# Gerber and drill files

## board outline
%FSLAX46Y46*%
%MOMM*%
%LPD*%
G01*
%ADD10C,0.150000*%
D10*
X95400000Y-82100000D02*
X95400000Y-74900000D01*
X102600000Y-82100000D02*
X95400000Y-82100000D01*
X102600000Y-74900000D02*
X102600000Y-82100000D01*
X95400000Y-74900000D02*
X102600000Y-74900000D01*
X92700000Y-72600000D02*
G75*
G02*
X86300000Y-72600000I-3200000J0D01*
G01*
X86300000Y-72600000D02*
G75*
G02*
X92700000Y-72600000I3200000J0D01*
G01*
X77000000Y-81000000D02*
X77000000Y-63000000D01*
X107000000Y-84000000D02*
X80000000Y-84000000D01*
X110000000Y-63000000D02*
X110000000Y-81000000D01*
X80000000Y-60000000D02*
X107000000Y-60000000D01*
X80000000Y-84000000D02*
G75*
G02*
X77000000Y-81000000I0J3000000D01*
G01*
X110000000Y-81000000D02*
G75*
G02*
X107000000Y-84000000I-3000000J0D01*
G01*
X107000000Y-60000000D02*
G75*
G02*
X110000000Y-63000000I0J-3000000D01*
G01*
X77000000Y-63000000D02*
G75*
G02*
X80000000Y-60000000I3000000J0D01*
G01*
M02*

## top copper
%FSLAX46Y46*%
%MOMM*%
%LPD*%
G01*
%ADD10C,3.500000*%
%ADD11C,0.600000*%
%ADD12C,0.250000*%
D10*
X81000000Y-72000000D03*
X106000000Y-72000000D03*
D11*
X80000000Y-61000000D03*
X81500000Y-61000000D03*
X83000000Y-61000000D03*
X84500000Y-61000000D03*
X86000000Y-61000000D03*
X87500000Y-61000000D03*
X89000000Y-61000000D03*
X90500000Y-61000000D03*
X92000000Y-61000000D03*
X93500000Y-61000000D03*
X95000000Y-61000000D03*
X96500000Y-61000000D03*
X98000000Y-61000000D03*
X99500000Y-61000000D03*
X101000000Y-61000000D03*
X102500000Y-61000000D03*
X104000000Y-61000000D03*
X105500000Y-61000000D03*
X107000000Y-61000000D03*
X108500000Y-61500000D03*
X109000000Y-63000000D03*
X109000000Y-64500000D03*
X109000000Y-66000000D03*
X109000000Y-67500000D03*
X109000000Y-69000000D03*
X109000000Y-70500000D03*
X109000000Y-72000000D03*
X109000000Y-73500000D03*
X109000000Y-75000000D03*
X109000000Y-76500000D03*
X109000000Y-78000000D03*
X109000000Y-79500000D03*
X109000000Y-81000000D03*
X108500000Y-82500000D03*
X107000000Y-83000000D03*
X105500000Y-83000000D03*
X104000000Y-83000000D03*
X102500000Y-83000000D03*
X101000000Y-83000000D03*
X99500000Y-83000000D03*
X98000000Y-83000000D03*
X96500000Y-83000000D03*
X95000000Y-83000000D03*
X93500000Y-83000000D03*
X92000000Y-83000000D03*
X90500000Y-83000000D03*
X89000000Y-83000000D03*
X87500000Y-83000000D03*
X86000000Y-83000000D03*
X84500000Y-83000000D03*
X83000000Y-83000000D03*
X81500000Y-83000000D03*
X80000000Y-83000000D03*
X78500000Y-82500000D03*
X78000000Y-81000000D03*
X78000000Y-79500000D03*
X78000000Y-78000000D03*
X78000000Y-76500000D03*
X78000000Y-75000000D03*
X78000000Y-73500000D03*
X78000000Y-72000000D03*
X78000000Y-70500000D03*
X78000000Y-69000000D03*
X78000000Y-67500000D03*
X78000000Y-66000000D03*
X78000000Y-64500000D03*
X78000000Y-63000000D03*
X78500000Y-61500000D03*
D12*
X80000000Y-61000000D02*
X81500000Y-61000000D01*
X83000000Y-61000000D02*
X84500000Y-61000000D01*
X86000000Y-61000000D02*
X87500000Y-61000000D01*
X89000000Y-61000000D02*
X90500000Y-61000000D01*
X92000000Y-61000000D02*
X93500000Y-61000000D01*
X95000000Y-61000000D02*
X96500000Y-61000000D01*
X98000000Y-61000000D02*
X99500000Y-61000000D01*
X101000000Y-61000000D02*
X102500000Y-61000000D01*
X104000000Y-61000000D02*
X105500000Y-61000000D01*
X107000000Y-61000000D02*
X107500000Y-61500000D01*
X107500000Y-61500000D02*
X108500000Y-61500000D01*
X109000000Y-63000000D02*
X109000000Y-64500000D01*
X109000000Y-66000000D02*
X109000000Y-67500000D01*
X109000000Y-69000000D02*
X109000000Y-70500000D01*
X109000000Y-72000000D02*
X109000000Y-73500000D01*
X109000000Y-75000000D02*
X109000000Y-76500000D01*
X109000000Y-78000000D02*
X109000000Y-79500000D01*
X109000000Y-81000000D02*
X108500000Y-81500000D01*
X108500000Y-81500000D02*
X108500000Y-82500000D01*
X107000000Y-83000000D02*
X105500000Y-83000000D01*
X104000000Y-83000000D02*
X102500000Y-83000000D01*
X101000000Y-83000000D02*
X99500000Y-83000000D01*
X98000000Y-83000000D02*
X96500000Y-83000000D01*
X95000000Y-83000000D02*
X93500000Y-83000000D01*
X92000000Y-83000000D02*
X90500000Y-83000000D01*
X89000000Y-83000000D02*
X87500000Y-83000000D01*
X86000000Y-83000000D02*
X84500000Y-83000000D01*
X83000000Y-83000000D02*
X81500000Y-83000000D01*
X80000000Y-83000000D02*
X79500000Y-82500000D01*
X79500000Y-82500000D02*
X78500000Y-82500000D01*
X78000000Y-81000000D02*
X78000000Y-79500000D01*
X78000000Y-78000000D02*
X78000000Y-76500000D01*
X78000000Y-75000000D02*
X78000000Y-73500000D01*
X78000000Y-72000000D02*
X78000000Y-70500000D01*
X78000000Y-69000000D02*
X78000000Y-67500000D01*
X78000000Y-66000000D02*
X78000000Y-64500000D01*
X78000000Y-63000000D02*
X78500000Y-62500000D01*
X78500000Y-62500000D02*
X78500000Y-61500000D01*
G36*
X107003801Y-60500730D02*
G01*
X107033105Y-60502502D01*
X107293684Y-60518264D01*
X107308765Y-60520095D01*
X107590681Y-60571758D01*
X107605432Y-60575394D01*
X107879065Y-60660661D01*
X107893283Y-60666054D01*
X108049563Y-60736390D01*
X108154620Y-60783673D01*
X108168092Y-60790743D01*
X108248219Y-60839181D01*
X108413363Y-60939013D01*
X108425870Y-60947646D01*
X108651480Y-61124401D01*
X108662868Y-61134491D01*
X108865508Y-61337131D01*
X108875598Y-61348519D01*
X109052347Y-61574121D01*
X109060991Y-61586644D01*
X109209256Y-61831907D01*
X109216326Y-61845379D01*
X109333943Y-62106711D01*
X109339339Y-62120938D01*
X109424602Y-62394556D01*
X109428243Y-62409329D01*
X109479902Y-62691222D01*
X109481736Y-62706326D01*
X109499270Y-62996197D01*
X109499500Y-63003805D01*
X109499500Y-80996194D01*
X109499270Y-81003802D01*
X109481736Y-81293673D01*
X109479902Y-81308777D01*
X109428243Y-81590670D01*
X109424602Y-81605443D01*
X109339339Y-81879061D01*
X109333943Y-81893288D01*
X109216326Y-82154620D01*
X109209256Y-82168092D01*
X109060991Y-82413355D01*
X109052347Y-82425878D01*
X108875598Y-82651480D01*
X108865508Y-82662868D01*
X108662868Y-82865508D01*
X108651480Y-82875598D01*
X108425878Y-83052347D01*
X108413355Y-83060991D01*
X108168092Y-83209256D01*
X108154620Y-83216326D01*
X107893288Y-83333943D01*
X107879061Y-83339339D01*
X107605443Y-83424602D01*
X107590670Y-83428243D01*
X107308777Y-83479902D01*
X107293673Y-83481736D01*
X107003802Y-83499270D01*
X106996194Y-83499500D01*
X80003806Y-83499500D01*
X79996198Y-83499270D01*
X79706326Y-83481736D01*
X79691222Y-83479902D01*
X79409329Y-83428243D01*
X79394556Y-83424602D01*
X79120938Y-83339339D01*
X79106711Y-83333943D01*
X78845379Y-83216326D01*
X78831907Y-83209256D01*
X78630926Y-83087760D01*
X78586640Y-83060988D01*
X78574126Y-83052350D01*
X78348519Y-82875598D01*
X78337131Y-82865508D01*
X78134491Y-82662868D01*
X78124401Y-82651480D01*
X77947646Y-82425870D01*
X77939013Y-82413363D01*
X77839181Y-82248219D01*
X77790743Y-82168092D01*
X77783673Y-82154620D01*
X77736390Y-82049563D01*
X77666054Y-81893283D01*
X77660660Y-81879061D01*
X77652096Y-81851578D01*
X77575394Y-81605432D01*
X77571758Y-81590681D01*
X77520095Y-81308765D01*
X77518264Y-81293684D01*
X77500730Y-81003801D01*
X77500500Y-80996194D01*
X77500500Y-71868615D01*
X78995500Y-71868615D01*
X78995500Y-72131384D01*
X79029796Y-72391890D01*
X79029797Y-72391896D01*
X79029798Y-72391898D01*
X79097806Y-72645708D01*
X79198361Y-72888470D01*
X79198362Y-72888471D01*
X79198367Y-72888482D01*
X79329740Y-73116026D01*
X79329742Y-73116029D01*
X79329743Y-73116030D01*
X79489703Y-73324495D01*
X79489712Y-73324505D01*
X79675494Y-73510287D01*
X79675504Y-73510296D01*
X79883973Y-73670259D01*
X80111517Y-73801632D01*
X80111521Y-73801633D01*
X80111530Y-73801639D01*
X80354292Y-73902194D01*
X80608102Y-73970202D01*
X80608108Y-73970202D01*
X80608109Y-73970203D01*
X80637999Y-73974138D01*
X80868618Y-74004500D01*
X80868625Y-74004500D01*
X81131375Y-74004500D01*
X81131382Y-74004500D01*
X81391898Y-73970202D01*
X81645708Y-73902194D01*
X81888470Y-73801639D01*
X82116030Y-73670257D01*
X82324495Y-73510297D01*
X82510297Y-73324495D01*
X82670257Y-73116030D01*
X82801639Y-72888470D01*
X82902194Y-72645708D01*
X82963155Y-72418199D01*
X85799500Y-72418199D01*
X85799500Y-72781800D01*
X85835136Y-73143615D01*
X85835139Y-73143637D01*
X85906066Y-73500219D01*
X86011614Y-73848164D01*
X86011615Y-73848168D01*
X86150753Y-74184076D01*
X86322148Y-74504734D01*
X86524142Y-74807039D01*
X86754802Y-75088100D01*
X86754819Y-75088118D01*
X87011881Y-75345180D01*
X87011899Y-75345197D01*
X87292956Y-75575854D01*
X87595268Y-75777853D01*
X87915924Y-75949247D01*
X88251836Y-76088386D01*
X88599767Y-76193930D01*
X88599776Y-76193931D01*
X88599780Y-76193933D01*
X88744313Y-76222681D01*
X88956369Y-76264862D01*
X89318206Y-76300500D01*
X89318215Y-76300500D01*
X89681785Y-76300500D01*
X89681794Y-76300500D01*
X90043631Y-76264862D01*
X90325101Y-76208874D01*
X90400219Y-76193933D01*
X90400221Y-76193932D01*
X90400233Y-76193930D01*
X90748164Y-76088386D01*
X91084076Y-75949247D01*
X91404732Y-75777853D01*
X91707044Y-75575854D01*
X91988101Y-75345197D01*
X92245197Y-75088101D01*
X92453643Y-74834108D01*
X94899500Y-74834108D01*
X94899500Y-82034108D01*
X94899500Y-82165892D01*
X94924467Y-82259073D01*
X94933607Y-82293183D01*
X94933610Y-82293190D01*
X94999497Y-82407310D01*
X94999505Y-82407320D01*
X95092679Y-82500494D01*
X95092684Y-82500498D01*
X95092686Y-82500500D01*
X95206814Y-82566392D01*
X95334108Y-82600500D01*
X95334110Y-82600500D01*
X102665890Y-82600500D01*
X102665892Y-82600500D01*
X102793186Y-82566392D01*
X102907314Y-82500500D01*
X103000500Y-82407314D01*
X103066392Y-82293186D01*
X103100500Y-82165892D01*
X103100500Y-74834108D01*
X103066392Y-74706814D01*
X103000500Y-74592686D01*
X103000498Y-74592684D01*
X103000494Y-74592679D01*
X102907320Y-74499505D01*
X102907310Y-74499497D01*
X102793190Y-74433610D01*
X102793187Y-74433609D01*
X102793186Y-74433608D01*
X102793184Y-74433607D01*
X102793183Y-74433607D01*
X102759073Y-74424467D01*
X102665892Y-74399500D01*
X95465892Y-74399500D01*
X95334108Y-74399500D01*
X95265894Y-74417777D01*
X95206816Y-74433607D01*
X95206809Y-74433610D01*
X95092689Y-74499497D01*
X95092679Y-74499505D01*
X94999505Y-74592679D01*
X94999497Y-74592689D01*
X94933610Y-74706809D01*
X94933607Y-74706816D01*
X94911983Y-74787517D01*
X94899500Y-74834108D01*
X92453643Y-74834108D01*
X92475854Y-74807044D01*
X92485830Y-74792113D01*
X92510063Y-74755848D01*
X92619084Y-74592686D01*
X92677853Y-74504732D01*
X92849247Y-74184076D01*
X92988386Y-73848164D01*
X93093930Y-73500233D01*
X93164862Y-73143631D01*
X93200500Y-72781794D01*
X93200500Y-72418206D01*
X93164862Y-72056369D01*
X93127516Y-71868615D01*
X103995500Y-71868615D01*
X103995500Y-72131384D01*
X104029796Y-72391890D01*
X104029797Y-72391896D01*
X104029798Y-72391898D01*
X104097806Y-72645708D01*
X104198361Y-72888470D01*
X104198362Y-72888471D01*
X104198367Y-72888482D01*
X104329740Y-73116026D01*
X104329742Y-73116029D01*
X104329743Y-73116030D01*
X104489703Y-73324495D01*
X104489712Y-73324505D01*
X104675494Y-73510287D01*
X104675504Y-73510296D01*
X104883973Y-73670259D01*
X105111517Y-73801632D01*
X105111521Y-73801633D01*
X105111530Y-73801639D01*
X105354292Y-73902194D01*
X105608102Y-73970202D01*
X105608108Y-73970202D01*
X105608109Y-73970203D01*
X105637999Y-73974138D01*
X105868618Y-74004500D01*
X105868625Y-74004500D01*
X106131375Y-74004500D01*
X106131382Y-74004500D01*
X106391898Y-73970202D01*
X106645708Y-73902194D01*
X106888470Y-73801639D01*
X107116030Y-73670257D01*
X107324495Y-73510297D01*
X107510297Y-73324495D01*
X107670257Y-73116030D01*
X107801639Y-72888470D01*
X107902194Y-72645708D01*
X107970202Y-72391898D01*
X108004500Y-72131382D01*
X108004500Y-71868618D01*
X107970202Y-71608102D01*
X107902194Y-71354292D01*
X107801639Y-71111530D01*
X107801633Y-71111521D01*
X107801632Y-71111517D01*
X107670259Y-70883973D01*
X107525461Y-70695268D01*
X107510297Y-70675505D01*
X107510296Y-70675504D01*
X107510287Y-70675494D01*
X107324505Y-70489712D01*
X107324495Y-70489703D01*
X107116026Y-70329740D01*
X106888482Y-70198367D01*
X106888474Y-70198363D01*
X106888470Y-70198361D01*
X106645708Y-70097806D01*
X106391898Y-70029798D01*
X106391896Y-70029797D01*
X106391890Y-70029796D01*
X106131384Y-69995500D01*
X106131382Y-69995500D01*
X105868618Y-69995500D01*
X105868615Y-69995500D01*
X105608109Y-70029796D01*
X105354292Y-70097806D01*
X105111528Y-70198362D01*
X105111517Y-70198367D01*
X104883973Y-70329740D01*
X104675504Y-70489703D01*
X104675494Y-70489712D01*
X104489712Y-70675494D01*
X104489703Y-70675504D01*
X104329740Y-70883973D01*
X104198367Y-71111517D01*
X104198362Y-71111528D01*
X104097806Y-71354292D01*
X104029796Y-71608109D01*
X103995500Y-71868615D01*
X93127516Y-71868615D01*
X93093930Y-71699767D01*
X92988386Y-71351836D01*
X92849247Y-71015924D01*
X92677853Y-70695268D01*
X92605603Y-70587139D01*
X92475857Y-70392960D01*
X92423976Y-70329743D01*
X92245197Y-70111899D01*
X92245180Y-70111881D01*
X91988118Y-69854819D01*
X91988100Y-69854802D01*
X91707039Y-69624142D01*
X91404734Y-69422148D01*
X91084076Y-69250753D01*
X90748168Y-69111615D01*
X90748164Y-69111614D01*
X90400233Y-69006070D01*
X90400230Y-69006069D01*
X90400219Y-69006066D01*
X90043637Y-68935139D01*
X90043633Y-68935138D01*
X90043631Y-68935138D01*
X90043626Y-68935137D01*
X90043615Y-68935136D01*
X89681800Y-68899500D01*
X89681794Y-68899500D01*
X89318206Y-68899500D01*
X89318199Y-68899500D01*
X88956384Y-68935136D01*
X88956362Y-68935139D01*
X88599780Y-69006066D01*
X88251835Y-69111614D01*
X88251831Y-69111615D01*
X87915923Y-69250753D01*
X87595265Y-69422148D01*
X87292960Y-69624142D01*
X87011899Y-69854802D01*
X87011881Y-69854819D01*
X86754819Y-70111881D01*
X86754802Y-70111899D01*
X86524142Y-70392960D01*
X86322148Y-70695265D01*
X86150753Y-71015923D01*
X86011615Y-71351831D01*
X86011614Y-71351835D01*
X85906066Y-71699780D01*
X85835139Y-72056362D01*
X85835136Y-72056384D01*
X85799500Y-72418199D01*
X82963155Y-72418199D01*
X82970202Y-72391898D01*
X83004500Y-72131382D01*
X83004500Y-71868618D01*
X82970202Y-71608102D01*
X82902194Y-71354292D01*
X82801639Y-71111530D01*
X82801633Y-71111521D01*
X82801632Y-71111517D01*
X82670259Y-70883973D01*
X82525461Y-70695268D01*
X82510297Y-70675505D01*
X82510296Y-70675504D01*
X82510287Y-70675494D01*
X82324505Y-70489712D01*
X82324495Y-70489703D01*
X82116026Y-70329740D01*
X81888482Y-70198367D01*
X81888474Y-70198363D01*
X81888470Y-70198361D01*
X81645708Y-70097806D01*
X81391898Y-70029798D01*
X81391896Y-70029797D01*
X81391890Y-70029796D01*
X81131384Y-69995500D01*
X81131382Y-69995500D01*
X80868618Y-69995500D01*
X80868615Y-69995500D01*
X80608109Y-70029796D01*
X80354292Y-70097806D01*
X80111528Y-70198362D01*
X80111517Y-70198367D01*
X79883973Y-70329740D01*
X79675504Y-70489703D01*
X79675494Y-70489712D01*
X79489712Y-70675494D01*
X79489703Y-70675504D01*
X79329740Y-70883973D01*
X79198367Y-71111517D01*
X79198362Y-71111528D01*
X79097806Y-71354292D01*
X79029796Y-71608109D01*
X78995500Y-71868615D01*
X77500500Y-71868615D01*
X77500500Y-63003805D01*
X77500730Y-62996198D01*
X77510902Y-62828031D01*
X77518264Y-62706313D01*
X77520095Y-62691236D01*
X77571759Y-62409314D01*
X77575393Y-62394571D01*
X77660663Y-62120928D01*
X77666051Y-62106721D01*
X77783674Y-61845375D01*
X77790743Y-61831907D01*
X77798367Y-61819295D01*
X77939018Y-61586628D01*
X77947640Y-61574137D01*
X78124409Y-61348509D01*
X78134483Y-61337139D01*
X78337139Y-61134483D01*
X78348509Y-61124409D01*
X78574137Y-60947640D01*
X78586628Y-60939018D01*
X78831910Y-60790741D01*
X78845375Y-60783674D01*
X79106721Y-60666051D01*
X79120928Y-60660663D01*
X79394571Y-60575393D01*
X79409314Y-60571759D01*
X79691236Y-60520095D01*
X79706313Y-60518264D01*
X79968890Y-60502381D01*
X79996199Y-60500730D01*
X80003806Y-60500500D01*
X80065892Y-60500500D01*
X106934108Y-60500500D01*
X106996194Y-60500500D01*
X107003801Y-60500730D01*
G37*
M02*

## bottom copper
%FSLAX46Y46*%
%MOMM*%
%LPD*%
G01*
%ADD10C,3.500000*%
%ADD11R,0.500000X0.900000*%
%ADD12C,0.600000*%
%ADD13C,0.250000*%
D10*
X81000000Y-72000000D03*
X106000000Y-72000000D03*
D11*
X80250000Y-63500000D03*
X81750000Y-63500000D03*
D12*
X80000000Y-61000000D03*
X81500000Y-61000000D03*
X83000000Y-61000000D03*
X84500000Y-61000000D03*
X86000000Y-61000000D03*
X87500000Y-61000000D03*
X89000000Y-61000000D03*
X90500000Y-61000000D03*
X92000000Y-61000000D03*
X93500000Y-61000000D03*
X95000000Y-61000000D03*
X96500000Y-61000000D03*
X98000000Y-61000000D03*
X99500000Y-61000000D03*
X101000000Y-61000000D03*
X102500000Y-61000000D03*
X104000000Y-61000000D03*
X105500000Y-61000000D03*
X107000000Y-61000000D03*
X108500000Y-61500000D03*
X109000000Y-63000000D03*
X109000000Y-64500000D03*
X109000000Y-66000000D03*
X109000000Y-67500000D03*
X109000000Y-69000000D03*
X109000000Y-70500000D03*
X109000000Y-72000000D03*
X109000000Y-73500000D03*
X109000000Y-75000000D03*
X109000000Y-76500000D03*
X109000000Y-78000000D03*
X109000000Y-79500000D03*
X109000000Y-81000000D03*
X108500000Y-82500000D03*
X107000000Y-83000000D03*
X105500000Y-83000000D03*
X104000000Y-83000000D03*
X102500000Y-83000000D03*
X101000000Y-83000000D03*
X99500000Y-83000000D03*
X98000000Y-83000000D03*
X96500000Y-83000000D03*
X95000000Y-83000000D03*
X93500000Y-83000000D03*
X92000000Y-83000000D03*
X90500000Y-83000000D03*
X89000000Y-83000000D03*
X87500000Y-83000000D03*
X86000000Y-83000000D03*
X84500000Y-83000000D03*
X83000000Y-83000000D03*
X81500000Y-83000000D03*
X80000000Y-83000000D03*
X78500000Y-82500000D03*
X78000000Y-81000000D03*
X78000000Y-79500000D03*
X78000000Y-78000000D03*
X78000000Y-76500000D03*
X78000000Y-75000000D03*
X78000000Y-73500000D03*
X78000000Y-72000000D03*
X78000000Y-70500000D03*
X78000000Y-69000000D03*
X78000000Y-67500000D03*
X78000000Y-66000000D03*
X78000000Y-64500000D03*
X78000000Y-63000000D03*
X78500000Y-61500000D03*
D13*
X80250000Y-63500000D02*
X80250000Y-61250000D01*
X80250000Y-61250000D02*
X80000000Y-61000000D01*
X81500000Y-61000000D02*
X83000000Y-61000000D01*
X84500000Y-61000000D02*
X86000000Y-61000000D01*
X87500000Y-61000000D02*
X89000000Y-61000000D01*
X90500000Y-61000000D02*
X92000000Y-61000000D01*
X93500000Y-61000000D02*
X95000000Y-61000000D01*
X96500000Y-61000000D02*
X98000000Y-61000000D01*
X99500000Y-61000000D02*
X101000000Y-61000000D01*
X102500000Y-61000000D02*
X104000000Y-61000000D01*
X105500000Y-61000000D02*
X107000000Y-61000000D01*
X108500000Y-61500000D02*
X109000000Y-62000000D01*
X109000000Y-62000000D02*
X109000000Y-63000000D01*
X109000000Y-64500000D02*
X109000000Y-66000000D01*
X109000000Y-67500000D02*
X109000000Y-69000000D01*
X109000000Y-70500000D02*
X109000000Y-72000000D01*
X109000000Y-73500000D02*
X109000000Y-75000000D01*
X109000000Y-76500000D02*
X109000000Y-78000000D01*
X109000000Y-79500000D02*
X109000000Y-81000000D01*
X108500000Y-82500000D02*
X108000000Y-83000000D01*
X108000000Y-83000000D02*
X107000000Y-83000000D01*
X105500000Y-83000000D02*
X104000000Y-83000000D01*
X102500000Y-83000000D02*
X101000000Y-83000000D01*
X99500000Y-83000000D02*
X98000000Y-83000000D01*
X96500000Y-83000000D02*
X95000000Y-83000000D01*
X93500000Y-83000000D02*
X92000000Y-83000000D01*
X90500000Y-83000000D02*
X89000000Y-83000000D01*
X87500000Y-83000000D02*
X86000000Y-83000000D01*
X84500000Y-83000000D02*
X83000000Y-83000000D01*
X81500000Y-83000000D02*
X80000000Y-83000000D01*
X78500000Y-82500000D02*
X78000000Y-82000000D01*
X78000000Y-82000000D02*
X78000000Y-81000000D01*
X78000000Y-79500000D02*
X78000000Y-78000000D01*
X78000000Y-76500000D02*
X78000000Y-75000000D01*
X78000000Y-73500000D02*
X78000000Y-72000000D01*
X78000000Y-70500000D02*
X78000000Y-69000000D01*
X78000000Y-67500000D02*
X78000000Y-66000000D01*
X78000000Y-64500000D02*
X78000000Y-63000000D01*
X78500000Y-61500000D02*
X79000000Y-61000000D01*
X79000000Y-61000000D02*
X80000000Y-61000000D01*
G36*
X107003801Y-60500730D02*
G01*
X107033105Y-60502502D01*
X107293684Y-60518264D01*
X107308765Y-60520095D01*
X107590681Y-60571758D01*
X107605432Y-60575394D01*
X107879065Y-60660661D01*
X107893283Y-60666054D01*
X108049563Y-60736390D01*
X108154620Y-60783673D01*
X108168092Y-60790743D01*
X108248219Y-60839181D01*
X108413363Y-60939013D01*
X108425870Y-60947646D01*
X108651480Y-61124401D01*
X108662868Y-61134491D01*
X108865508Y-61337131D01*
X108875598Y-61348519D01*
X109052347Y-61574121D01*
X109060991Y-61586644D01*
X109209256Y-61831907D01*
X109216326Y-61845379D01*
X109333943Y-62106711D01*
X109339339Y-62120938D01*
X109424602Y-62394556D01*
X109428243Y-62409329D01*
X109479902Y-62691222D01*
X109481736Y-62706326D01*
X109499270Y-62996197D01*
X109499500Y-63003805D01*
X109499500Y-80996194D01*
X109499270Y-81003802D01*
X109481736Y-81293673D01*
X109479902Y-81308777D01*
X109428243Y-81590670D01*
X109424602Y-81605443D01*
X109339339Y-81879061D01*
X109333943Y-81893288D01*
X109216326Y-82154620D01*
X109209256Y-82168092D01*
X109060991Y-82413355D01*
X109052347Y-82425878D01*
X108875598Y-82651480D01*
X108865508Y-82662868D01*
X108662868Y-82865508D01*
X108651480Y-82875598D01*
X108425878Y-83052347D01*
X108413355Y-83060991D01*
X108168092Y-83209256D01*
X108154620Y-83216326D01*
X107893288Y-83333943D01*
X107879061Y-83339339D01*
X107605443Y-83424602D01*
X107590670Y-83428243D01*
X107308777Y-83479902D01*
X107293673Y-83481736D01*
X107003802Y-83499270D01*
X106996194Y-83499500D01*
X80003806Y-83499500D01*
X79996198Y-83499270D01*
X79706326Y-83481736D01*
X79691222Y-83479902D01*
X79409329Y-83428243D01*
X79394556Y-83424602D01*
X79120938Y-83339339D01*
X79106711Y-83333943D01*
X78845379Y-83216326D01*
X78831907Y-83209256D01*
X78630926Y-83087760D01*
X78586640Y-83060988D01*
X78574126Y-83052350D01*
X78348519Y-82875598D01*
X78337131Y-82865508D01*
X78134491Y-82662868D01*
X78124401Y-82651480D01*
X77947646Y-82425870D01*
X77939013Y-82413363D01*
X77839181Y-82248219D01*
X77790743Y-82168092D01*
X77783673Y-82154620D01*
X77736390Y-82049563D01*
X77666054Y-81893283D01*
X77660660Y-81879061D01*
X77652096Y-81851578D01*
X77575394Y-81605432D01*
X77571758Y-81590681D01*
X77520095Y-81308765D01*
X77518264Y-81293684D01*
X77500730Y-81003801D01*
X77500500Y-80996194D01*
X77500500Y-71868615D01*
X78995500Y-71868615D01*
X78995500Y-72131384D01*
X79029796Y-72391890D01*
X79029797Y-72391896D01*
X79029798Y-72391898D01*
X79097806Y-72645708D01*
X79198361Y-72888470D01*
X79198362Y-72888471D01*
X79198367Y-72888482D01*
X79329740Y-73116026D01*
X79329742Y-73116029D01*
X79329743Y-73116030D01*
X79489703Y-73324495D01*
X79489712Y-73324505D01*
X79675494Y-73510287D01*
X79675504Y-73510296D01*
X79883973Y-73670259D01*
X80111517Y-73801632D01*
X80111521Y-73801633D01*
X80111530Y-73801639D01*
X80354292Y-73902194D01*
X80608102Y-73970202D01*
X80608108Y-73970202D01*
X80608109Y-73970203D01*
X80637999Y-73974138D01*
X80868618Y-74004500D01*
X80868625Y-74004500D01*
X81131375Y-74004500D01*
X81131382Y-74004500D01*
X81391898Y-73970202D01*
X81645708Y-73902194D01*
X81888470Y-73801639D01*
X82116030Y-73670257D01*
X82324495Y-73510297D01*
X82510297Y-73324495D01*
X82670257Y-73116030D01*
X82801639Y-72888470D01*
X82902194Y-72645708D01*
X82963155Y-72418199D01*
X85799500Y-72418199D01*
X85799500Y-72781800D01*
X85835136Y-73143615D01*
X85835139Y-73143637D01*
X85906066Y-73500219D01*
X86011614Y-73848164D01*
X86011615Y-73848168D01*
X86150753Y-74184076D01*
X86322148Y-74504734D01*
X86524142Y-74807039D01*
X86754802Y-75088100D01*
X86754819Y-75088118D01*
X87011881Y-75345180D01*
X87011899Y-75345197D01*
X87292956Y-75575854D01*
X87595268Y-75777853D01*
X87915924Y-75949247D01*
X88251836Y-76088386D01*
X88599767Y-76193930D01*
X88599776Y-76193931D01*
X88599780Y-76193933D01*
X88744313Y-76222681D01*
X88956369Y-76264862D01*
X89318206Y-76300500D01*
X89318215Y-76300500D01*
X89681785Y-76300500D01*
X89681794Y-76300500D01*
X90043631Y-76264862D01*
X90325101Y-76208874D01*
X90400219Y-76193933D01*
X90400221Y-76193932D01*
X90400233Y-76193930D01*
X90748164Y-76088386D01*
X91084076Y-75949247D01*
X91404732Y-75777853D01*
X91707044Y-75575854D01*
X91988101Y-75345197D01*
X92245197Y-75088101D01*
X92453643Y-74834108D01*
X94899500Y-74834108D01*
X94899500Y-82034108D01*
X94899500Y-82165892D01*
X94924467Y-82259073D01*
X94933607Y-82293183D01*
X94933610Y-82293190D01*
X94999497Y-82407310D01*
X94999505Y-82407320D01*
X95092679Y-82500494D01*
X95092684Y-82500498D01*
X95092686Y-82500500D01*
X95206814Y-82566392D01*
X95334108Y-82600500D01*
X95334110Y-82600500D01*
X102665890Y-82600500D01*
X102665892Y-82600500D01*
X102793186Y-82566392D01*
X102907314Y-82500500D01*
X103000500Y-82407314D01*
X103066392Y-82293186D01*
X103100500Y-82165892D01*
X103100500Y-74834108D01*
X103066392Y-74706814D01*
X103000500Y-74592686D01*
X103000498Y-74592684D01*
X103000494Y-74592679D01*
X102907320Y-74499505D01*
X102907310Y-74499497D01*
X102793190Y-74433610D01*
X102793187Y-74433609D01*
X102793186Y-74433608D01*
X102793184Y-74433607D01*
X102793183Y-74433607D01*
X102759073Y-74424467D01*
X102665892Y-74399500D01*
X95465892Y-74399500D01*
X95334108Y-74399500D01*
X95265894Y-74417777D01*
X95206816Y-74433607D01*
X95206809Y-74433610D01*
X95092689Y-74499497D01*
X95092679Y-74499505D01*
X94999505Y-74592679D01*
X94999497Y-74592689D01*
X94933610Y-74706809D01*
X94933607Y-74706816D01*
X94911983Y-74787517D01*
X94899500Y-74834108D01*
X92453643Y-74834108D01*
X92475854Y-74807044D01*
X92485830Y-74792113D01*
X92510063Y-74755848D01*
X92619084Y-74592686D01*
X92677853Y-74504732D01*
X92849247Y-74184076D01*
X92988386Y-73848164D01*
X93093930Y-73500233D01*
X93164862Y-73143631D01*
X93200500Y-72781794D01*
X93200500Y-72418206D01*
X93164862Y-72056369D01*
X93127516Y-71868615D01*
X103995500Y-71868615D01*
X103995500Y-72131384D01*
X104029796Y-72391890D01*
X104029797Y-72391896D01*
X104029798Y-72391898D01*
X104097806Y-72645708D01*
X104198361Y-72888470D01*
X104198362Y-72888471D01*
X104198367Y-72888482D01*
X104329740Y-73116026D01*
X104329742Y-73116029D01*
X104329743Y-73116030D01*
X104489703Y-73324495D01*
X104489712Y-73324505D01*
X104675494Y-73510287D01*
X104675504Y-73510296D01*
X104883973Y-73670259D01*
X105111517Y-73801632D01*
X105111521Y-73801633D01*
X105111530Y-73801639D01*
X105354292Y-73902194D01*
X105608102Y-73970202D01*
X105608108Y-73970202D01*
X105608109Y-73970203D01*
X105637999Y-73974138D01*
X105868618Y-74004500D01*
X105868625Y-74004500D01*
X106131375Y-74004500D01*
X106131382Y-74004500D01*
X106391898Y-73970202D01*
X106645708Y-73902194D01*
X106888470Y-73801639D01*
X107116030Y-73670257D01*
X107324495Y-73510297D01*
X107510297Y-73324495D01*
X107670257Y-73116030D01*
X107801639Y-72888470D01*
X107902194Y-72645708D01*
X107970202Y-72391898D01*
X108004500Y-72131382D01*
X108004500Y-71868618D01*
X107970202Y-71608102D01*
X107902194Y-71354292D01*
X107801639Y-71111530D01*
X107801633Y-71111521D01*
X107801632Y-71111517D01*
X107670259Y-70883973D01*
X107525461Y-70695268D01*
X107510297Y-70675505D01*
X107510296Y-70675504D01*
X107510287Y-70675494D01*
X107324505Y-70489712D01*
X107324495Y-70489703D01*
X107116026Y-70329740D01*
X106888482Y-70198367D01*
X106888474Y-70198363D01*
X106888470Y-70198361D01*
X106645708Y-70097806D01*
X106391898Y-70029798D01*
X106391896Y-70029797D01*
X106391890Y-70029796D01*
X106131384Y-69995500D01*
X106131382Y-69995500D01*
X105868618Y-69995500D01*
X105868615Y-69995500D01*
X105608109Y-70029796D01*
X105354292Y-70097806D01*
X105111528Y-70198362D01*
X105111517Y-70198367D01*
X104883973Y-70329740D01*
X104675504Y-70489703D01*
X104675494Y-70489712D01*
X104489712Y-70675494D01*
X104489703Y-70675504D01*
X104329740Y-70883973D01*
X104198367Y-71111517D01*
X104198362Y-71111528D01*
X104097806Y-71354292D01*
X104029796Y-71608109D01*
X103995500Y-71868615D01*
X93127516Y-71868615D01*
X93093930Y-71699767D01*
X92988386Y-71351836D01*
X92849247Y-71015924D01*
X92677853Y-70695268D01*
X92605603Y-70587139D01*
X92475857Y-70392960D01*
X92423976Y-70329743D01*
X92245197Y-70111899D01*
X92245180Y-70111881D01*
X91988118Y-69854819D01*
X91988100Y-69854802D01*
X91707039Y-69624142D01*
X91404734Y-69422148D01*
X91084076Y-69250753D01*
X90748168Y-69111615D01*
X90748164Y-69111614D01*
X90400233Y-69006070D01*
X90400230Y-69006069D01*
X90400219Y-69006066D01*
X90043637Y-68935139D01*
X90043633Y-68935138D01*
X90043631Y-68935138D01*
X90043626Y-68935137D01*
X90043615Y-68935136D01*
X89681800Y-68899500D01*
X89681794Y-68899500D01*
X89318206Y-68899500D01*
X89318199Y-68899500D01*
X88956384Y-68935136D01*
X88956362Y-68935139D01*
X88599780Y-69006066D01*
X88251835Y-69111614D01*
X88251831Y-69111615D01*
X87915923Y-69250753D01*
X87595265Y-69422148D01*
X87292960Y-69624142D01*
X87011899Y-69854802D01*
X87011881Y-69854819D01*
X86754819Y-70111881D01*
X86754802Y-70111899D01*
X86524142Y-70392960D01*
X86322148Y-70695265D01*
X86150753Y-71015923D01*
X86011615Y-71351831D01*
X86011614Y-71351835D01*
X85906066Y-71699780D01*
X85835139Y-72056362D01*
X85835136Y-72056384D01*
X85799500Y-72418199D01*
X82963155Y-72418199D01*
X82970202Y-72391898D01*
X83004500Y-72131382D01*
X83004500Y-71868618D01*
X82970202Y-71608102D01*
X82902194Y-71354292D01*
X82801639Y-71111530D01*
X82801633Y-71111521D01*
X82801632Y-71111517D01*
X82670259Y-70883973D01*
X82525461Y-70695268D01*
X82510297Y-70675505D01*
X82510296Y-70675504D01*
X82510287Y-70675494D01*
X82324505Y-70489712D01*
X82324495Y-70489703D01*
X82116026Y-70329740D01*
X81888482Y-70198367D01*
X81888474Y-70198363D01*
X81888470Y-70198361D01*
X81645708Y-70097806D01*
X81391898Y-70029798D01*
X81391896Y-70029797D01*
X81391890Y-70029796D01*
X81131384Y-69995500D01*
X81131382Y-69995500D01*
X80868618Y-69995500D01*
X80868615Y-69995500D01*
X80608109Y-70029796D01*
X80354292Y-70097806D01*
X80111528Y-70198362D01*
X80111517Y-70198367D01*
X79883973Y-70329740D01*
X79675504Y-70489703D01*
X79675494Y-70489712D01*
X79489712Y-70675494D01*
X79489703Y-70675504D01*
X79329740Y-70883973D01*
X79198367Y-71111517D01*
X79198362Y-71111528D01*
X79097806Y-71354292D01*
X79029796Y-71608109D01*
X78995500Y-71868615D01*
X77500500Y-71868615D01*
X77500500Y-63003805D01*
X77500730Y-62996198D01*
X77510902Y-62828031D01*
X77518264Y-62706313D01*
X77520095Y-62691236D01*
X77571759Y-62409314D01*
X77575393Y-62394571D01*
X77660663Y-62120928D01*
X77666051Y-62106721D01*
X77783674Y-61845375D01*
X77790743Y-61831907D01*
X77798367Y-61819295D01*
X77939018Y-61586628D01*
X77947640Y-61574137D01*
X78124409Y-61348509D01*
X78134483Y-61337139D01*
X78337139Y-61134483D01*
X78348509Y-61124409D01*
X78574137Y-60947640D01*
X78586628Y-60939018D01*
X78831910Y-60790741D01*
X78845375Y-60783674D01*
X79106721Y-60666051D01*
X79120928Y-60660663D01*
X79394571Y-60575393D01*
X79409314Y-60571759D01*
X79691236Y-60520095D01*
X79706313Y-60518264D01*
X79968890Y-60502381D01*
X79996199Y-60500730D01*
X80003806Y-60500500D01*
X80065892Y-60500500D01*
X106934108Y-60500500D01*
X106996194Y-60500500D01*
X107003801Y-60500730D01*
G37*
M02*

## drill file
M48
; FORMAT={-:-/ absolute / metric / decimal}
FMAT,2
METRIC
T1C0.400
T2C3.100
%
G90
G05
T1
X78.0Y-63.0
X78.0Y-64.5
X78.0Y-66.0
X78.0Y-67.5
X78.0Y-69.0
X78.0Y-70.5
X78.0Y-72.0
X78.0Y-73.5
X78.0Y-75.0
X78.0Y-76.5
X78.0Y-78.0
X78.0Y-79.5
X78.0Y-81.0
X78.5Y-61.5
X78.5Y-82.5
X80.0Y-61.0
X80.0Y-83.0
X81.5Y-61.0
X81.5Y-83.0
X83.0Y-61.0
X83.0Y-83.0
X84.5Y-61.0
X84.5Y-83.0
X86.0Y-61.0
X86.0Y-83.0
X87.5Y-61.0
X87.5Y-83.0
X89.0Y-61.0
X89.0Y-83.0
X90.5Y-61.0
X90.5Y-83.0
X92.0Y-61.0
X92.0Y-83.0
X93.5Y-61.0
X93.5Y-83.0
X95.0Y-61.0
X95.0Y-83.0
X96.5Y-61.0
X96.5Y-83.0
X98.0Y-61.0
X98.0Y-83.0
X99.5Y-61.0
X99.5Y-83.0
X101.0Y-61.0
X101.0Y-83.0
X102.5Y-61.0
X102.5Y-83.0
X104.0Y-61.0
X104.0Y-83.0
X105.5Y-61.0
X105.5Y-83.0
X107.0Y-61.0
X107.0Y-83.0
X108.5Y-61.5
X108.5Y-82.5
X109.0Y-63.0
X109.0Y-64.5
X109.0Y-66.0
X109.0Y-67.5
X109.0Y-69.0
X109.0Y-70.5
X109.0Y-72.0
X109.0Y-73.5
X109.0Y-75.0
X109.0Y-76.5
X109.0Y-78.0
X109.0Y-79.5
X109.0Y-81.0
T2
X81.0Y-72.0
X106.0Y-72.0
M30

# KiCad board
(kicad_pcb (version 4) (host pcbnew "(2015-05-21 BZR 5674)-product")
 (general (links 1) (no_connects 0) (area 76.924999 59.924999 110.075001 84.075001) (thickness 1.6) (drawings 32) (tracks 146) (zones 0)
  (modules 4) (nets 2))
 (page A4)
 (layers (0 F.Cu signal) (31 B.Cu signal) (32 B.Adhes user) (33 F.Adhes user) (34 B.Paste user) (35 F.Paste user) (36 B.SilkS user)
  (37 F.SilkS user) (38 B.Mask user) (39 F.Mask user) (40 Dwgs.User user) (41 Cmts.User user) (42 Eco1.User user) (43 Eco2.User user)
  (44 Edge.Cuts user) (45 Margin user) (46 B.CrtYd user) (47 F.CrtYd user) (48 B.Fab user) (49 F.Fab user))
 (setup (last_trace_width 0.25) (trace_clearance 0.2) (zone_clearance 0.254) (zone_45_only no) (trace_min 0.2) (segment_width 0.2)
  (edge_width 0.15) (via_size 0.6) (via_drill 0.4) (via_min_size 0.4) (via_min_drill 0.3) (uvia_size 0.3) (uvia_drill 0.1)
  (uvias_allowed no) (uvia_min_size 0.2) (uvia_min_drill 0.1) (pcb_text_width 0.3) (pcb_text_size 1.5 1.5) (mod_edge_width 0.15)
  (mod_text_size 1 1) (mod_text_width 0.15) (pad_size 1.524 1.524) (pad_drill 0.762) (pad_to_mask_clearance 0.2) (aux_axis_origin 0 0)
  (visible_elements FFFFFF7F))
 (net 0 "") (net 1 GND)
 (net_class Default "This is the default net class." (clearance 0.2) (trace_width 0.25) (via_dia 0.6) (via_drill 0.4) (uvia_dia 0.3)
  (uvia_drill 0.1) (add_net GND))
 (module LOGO (layer F.Cu) (at 104.5 66)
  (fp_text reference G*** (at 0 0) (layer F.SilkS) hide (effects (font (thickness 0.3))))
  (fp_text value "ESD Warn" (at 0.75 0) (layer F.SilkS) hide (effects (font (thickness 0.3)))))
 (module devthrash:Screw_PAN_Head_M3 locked (layer B.Cu) (at 81 72)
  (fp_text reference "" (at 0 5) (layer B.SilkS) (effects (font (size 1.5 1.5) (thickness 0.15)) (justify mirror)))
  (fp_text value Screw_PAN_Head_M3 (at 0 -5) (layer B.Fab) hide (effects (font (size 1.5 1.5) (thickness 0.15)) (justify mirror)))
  (pad "" np_thru_hole circle (at 0 0) (size 3.5 3.5) (drill 3.1) (layers *.Cu *.Mask B.SilkS)))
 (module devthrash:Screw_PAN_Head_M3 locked (layer B.Cu) (at 106 72)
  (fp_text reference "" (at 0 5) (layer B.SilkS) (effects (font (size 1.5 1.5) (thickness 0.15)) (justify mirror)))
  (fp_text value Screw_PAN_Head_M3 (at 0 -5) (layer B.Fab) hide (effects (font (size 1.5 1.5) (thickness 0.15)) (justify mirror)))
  (pad "" np_thru_hole circle (at 0 0) (size 3.5 3.5) (drill 3.1) (layers *.Cu *.Mask B.SilkS)))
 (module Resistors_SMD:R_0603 (layer B.Cu) (at 81 63.5) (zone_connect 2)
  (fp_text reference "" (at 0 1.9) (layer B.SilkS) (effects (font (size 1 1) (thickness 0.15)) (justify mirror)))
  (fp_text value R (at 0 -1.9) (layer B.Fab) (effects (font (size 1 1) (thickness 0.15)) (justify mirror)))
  (pad 1 smd rect (at -0.75 0) (size 0.5 0.9) (layers B.Cu B.Paste B.Mask) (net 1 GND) (zone_connect 2))
  (pad 2 smd rect (at 0.75 0) (size 0.5 0.9) (layers B.Cu B.Paste B.Mask) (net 1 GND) (zone_connect 2)))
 (gr_line (start 95.4 82.1) (end 95.4 74.9) (angle 90) (layer Edge.Cuts) (width 0.15))
 (gr_line (start 102.6 82.1) (end 95.4 82.1) (angle 90) (layer Edge.Cuts) (width 0.15))
 (gr_line (start 102.6 74.9) (end 102.6 82.1) (angle 90) (layer Edge.Cuts) (width 0.15))
 (gr_line (start 95.4 74.9) (end 102.6 74.9) (angle 90) (layer Edge.Cuts) (width 0.15))
 (gr_circle (center 89.5 72.6) (end 92.7 72.6) (layer Edge.Cuts) (width 0.15))
 (gr_line (start 77 81) (end 77 63) (angle 90) (layer Edge.Cuts) (width 0.15))
 (gr_line (start 107 84) (end 80 84) (angle 90) (layer Edge.Cuts) (width 0.15))
 (gr_line (start 110 63) (end 110 81) (angle 90) (layer Edge.Cuts) (width 0.15))
 (gr_line (start 80 60) (end 107 60) (angle 90) (layer Edge.Cuts) (width 0.15))
 (gr_arc (start 80 81) (end 80 84) (angle 90) (layer Edge.Cuts) (width 0.15))
 (gr_arc (start 107 81) (end 110 81) (angle 90) (layer Edge.Cuts) (width 0.15))
 (gr_arc (start 107 63) (end 107 60) (angle 90) (layer Edge.Cuts) (width 0.15))
 (gr_arc (start 80 63) (end 77 63) (angle 90) (layer Edge.Cuts) (width 0.15))
 (segment (start 80.25 63.5) (end 80.25 61.25) (width 0.25) (layer B.Cu) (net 1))
 (segment (start 80.25 61.25) (end 80 61) (width 0.25) (layer B.Cu) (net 1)) (via (at 80 61) (size 0.6) (layers F.Cu B.Cu) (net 1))
 (segment (start 80 61) (end 81.5 61) (width 0.25) (layer F.Cu) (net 1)) (via (at 81.5 61) (size 0.6) (layers F.Cu B.Cu) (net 1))
 (segment (start 81.5 61) (end 83 61) (width 0.25) (layer B.Cu) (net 1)) (via (at 83 61) (size 0.6) (layers F.Cu B.Cu) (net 1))
 (segment (start 83 61) (end 84.5 61) (width 0.25) (layer F.Cu) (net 1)) (via (at 84.5 61) (size 0.6) (layers F.Cu B.Cu) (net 1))
 (segment (start 84.5 61) (end 86 61) (width 0.25) (layer B.Cu) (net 1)) (via (at 86 61) (size 0.6) (layers F.Cu B.Cu) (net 1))
 (segment (start 86 61) (end 87.5 61) (width 0.25) (layer F.Cu) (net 1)) (via (at 87.5 61) (size 0.6) (layers F.Cu B.Cu) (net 1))
 (segment (start 87.5 61) (end 89 61) (width 0.25) (layer B.Cu) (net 1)) (via (at 89 61) (size 0.6) (layers F.Cu B.Cu) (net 1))
 (segment (start 89 61) (end 90.5 61) (width 0.25) (layer F.Cu) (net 1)) (via (at 90.5 61) (size 0.6) (layers F.Cu B.Cu) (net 1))
 (segment (start 90.5 61) (end 92 61) (width 0.25) (layer B.Cu) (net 1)) (via (at 92 61) (size 0.6) (layers F.Cu B.Cu) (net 1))
 (segment (start 92 61) (end 93.5 61) (width 0.25) (layer F.Cu) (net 1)) (via (at 93.5 61) (size 0.6) (layers F.Cu B.Cu) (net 1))
 (segment (start 93.5 61) (end 95 61) (width 0.25) (layer B.Cu) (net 1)) (via (at 95 61) (size 0.6) (layers F.Cu B.Cu) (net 1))
 (segment (start 95 61) (end 96.5 61) (width 0.25) (layer F.Cu) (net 1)) (via (at 96.5 61) (size 0.6) (layers F.Cu B.Cu) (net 1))
 (segment (start 96.5 61) (end 98 61) (width 0.25) (layer B.Cu) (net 1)) (via (at 98 61) (size 0.6) (layers F.Cu B.Cu) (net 1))
 (segment (start 98 61) (end 99.5 61) (width 0.25) (layer F.Cu) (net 1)) (via (at 99.5 61) (size 0.6) (layers F.Cu B.Cu) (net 1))
 (segment (start 99.5 61) (end 101 61) (width 0.25) (layer B.Cu) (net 1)) (via (at 101 61) (size 0.6) (layers F.Cu B.Cu) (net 1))
 (segment (start 101 61) (end 102.5 61) (width 0.25) (layer F.Cu) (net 1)) (via (at 102.5 61) (size 0.6) (layers F.Cu B.Cu) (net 1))
 (segment (start 102.5 61) (end 104 61) (width 0.25) (layer B.Cu) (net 1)) (via (at 104 61) (size 0.6) (layers F.Cu B.Cu) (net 1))
 (segment (start 104 61) (end 105.5 61) (width 0.25) (layer F.Cu) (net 1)) (via (at 105.5 61) (size 0.6) (layers F.Cu B.Cu) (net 1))
 (segment (start 105.5 61) (end 107 61) (width 0.25) (layer B.Cu) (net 1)) (via (at 107 61) (size 0.6) (layers F.Cu B.Cu) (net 1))
 (segment (start 107 61) (end 107.5 61.5) (width 0.25) (layer F.Cu) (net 1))
 (segment (start 107.5 61.5) (end 108.5 61.5) (width 0.25) (layer F.Cu) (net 1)) (via (at 108.5 61.5) (size 0.6) (layers F.Cu B.Cu) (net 1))
 (segment (start 108.5 61.5) (end 109 62) (width 0.25) (layer B.Cu) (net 1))
 (segment (start 109 62) (end 109 63) (width 0.25) (layer B.Cu) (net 1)) (via (at 109 63) (size 0.6) (layers F.Cu B.Cu) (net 1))
 (segment (start 109 63) (end 109 64.5) (width 0.25) (layer F.Cu) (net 1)) (via (at 109 64.5) (size 0.6) (layers F.Cu B.Cu) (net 1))
 (segment (start 109 64.5) (end 109 66) (width 0.25) (layer B.Cu) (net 1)) (via (at 109 66) (size 0.6) (layers F.Cu B.Cu) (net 1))
 (segment (start 109 66) (end 109 67.5) (width 0.25) (layer F.Cu) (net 1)) (via (at 109 67.5) (size 0.6) (layers F.Cu B.Cu) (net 1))
 (segment (start 109 67.5) (end 109 69) (width 0.25) (layer B.Cu) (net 1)) (via (at 109 69) (size 0.6) (layers F.Cu B.Cu) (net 1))
 (segment (start 109 69) (end 109 70.5) (width 0.25) (layer F.Cu) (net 1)) (via (at 109 70.5) (size 0.6) (layers F.Cu B.Cu) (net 1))
 (segment (start 109 70.5) (end 109 72) (width 0.25) (layer B.Cu) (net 1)) (via (at 109 72) (size 0.6) (layers F.Cu B.Cu) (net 1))
 (segment (start 109 72) (end 109 73.5) (width 0.25) (layer F.Cu) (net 1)) (via (at 109 73.5) (size 0.6) (layers F.Cu B.Cu) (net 1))
 (segment (start 109 73.5) (end 109 75) (width 0.25) (layer B.Cu) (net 1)) (via (at 109 75) (size 0.6) (layers F.Cu B.Cu) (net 1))
 (segment (start 109 75) (end 109 76.5) (width 0.25) (layer F.Cu) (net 1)) (via (at 109 76.5) (size 0.6) (layers F.Cu B.Cu) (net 1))
 (segment (start 109 76.5) (end 109 78) (width 0.25) (layer B.Cu) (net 1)) (via (at 109 78) (size 0.6) (layers F.Cu B.Cu) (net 1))
 (segment (start 109 78) (end 109 79.5) (width 0.25) (layer F.Cu) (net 1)) (via (at 109 79.5) (size 0.6) (layers F.Cu B.Cu) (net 1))
 (segment (start 109 79.5) (end 109 81) (width 0.25) (layer B.Cu) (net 1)) (via (at 109 81) (size 0.6) (layers F.Cu B.Cu) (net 1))
 (segment (start 109 81) (end 108.5 81.5) (width 0.25) (layer F.Cu) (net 1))
 (segment (start 108.5 81.5) (end 108.5 82.5) (width 0.25) (layer F.Cu) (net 1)) (via (at 108.5 82.5) (size 0.6) (layers F.Cu B.Cu) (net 1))
 (segment (start 108.5 82.5) (end 108 83) (width 0.25) (layer B.Cu) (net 1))
 (segment (start 108 83) (end 107 83) (width 0.25) (layer B.Cu) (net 1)) (via (at 107 83) (size 0.6) (layers F.Cu B.Cu) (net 1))
 (segment (start 107 83) (end 105.5 83) (width 0.25) (layer F.Cu) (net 1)) (via (at 105.5 83) (size 0.6) (layers F.Cu B.Cu) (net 1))
 (segment (start 105.5 83) (end 104 83) (width 0.25) (layer B.Cu) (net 1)) (via (at 104 83) (size 0.6) (layers F.Cu B.Cu) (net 1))
 (segment (start 104 83) (end 102.5 83) (width 0.25) (layer F.Cu) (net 1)) (via (at 102.5 83) (size 0.6) (layers F.Cu B.Cu) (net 1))
 (segment (start 102.5 83) (end 101 83) (width 0.25) (layer B.Cu) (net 1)) (via (at 101 83) (size 0.6) (layers F.Cu B.Cu) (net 1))
 (segment (start 101 83) (end 99.5 83) (width 0.25) (layer F.Cu) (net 1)) (via (at 99.5 83) (size 0.6) (layers F.Cu B.Cu) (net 1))
 (segment (start 99.5 83) (end 98 83) (width 0.25) (layer B.Cu) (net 1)) (via (at 98 83) (size 0.6) (layers F.Cu B.Cu) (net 1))
 (segment (start 98 83) (end 96.5 83) (width 0.25) (layer F.Cu) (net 1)) (via (at 96.5 83) (size 0.6) (layers F.Cu B.Cu) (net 1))
 (segment (start 96.5 83) (end 95 83) (width 0.25) (layer B.Cu) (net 1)) (via (at 95 83) (size 0.6) (layers F.Cu B.Cu) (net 1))
 (segment (start 95 83) (end 93.5 83) (width 0.25) (layer F.Cu) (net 1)) (via (at 93.5 83) (size 0.6) (layers F.Cu B.Cu) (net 1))
 (segment (start 93.5 83) (end 92 83) (width 0.25) (layer B.Cu) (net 1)) (via (at 92 83) (size 0.6) (layers F.Cu B.Cu) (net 1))
 (segment (start 92 83) (end 90.5 83) (width 0.25) (layer F.Cu) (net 1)) (via (at 90.5 83) (size 0.6) (layers F.Cu B.Cu) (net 1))
 (segment (start 90.5 83) (end 89 83) (width 0.25) (layer B.Cu) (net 1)) (via (at 89 83) (size 0.6) (layers F.Cu B.Cu) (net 1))
 (segment (start 89 83) (end 87.5 83) (width 0.25) (layer F.Cu) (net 1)) (via (at 87.5 83) (size 0.6) (layers F.Cu B.Cu) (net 1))
 (segment (start 87.5 83) (end 86 83) (width 0.25) (layer B.Cu) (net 1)) (via (at 86 83) (size 0.6) (layers F.Cu B.Cu) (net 1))
 (segment (start 86 83) (end 84.5 83) (width 0.25) (layer F.Cu) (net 1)) (via (at 84.5 83) (size 0.6) (layers F.Cu B.Cu) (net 1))
 (segment (start 84.5 83) (end 83 83) (width 0.25) (layer B.Cu) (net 1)) (via (at 83 83) (size 0.6) (layers F.Cu B.Cu) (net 1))
 (segment (start 83 83) (end 81.5 83) (width 0.25) (layer F.Cu) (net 1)) (via (at 81.5 83) (size 0.6) (layers F.Cu B.Cu) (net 1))
 (segment (start 81.5 83) (end 80 83) (width 0.25) (layer B.Cu) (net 1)) (via (at 80 83) (size 0.6) (layers F.Cu B.Cu) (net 1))
 (segment (start 80 83) (end 79.5 82.5) (width 0.25) (layer F.Cu) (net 1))
 (segment (start 79.5 82.5) (end 78.5 82.5) (width 0.25) (layer F.Cu) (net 1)) (via (at 78.5 82.5) (size 0.6) (layers F.Cu B.Cu) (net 1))
 (segment (start 78.5 82.5) (end 78 82) (width 0.25) (layer B.Cu) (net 1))
 (segment (start 78 82) (end 78 81) (width 0.25) (layer B.Cu) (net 1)) (via (at 78 81) (size 0.6) (layers F.Cu B.Cu) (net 1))
 (segment (start 78 81) (end 78 79.5) (width 0.25) (layer F.Cu) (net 1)) (via (at 78 79.5) (size 0.6) (layers F.Cu B.Cu) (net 1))
 (segment (start 78 79.5) (end 78 78) (width 0.25) (layer B.Cu) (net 1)) (via (at 78 78) (size 0.6) (layers F.Cu B.Cu) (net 1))
 (segment (start 78 78) (end 78 76.5) (width 0.25) (layer F.Cu) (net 1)) (via (at 78 76.5) (size 0.6) (layers F.Cu B.Cu) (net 1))
 (segment (start 78 76.5) (end 78 75) (width 0.25) (layer B.Cu) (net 1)) (via (at 78 75) (size 0.6) (layers F.Cu B.Cu) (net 1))
 (segment (start 78 75) (end 78 73.5) (width 0.25) (layer F.Cu) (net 1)) (via (at 78 73.5) (size 0.6) (layers F.Cu B.Cu) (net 1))
 (segment (start 78 73.5) (end 78 72) (width 0.25) (layer B.Cu) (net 1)) (via (at 78 72) (size 0.6) (layers F.Cu B.Cu) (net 1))
 (segment (start 78 72) (end 78 70.5) (width 0.25) (layer F.Cu) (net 1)) (via (at 78 70.5) (size 0.6) (layers F.Cu B.Cu) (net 1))
 (segment (start 78 70.5) (end 78 69) (width 0.25) (layer B.Cu) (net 1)) (via (at 78 69) (size 0.6) (layers F.Cu B.Cu) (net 1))
 (segment (start 78 69) (end 78 67.5) (width 0.25) (layer F.Cu) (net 1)) (via (at 78 67.5) (size 0.6) (layers F.Cu B.Cu) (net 1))
 (segment (start 78 67.5) (end 78 66) (width 0.25) (layer B.Cu) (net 1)) (via (at 78 66) (size 0.6) (layers F.Cu B.Cu) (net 1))
 (segment (start 78 66) (end 78 64.5) (width 0.25) (layer F.Cu) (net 1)) (via (at 78 64.5) (size 0.6) (layers F.Cu B.Cu) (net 1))
 (segment (start 78 64.5) (end 78 63) (width 0.25) (layer B.Cu) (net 1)) (via (at 78 63) (size 0.6) (layers F.Cu B.Cu) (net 1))
 (segment (start 78 63) (end 78.5 62.5) (width 0.25) (layer F.Cu) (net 1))
 (segment (start 78.5 62.5) (end 78.5 61.5) (width 0.25) (layer F.Cu) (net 1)) (via (at 78.5 61.5) (size 0.6) (layers F.Cu B.Cu) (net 1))
 (segment (start 78.5 61.5) (end 79 61) (width 0.25) (layer B.Cu) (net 1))
 (segment (start 79 61) (end 80 61) (width 0.25) (layer B.Cu) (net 1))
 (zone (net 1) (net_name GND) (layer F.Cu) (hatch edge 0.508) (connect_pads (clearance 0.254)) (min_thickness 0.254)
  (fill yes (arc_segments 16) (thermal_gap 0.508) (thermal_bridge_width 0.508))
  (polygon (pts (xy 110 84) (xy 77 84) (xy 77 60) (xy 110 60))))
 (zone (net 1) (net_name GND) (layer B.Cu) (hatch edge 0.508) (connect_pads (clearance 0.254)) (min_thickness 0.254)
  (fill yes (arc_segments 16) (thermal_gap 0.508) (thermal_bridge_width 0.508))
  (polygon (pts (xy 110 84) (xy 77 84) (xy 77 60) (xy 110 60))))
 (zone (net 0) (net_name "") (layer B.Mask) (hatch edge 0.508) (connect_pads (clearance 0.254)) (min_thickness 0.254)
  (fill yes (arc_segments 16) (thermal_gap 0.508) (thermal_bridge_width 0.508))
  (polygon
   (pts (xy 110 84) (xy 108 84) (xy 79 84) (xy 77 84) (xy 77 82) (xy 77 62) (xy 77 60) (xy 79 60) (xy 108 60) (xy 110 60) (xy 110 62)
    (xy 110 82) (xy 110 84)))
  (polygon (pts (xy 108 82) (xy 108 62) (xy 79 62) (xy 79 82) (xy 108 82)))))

